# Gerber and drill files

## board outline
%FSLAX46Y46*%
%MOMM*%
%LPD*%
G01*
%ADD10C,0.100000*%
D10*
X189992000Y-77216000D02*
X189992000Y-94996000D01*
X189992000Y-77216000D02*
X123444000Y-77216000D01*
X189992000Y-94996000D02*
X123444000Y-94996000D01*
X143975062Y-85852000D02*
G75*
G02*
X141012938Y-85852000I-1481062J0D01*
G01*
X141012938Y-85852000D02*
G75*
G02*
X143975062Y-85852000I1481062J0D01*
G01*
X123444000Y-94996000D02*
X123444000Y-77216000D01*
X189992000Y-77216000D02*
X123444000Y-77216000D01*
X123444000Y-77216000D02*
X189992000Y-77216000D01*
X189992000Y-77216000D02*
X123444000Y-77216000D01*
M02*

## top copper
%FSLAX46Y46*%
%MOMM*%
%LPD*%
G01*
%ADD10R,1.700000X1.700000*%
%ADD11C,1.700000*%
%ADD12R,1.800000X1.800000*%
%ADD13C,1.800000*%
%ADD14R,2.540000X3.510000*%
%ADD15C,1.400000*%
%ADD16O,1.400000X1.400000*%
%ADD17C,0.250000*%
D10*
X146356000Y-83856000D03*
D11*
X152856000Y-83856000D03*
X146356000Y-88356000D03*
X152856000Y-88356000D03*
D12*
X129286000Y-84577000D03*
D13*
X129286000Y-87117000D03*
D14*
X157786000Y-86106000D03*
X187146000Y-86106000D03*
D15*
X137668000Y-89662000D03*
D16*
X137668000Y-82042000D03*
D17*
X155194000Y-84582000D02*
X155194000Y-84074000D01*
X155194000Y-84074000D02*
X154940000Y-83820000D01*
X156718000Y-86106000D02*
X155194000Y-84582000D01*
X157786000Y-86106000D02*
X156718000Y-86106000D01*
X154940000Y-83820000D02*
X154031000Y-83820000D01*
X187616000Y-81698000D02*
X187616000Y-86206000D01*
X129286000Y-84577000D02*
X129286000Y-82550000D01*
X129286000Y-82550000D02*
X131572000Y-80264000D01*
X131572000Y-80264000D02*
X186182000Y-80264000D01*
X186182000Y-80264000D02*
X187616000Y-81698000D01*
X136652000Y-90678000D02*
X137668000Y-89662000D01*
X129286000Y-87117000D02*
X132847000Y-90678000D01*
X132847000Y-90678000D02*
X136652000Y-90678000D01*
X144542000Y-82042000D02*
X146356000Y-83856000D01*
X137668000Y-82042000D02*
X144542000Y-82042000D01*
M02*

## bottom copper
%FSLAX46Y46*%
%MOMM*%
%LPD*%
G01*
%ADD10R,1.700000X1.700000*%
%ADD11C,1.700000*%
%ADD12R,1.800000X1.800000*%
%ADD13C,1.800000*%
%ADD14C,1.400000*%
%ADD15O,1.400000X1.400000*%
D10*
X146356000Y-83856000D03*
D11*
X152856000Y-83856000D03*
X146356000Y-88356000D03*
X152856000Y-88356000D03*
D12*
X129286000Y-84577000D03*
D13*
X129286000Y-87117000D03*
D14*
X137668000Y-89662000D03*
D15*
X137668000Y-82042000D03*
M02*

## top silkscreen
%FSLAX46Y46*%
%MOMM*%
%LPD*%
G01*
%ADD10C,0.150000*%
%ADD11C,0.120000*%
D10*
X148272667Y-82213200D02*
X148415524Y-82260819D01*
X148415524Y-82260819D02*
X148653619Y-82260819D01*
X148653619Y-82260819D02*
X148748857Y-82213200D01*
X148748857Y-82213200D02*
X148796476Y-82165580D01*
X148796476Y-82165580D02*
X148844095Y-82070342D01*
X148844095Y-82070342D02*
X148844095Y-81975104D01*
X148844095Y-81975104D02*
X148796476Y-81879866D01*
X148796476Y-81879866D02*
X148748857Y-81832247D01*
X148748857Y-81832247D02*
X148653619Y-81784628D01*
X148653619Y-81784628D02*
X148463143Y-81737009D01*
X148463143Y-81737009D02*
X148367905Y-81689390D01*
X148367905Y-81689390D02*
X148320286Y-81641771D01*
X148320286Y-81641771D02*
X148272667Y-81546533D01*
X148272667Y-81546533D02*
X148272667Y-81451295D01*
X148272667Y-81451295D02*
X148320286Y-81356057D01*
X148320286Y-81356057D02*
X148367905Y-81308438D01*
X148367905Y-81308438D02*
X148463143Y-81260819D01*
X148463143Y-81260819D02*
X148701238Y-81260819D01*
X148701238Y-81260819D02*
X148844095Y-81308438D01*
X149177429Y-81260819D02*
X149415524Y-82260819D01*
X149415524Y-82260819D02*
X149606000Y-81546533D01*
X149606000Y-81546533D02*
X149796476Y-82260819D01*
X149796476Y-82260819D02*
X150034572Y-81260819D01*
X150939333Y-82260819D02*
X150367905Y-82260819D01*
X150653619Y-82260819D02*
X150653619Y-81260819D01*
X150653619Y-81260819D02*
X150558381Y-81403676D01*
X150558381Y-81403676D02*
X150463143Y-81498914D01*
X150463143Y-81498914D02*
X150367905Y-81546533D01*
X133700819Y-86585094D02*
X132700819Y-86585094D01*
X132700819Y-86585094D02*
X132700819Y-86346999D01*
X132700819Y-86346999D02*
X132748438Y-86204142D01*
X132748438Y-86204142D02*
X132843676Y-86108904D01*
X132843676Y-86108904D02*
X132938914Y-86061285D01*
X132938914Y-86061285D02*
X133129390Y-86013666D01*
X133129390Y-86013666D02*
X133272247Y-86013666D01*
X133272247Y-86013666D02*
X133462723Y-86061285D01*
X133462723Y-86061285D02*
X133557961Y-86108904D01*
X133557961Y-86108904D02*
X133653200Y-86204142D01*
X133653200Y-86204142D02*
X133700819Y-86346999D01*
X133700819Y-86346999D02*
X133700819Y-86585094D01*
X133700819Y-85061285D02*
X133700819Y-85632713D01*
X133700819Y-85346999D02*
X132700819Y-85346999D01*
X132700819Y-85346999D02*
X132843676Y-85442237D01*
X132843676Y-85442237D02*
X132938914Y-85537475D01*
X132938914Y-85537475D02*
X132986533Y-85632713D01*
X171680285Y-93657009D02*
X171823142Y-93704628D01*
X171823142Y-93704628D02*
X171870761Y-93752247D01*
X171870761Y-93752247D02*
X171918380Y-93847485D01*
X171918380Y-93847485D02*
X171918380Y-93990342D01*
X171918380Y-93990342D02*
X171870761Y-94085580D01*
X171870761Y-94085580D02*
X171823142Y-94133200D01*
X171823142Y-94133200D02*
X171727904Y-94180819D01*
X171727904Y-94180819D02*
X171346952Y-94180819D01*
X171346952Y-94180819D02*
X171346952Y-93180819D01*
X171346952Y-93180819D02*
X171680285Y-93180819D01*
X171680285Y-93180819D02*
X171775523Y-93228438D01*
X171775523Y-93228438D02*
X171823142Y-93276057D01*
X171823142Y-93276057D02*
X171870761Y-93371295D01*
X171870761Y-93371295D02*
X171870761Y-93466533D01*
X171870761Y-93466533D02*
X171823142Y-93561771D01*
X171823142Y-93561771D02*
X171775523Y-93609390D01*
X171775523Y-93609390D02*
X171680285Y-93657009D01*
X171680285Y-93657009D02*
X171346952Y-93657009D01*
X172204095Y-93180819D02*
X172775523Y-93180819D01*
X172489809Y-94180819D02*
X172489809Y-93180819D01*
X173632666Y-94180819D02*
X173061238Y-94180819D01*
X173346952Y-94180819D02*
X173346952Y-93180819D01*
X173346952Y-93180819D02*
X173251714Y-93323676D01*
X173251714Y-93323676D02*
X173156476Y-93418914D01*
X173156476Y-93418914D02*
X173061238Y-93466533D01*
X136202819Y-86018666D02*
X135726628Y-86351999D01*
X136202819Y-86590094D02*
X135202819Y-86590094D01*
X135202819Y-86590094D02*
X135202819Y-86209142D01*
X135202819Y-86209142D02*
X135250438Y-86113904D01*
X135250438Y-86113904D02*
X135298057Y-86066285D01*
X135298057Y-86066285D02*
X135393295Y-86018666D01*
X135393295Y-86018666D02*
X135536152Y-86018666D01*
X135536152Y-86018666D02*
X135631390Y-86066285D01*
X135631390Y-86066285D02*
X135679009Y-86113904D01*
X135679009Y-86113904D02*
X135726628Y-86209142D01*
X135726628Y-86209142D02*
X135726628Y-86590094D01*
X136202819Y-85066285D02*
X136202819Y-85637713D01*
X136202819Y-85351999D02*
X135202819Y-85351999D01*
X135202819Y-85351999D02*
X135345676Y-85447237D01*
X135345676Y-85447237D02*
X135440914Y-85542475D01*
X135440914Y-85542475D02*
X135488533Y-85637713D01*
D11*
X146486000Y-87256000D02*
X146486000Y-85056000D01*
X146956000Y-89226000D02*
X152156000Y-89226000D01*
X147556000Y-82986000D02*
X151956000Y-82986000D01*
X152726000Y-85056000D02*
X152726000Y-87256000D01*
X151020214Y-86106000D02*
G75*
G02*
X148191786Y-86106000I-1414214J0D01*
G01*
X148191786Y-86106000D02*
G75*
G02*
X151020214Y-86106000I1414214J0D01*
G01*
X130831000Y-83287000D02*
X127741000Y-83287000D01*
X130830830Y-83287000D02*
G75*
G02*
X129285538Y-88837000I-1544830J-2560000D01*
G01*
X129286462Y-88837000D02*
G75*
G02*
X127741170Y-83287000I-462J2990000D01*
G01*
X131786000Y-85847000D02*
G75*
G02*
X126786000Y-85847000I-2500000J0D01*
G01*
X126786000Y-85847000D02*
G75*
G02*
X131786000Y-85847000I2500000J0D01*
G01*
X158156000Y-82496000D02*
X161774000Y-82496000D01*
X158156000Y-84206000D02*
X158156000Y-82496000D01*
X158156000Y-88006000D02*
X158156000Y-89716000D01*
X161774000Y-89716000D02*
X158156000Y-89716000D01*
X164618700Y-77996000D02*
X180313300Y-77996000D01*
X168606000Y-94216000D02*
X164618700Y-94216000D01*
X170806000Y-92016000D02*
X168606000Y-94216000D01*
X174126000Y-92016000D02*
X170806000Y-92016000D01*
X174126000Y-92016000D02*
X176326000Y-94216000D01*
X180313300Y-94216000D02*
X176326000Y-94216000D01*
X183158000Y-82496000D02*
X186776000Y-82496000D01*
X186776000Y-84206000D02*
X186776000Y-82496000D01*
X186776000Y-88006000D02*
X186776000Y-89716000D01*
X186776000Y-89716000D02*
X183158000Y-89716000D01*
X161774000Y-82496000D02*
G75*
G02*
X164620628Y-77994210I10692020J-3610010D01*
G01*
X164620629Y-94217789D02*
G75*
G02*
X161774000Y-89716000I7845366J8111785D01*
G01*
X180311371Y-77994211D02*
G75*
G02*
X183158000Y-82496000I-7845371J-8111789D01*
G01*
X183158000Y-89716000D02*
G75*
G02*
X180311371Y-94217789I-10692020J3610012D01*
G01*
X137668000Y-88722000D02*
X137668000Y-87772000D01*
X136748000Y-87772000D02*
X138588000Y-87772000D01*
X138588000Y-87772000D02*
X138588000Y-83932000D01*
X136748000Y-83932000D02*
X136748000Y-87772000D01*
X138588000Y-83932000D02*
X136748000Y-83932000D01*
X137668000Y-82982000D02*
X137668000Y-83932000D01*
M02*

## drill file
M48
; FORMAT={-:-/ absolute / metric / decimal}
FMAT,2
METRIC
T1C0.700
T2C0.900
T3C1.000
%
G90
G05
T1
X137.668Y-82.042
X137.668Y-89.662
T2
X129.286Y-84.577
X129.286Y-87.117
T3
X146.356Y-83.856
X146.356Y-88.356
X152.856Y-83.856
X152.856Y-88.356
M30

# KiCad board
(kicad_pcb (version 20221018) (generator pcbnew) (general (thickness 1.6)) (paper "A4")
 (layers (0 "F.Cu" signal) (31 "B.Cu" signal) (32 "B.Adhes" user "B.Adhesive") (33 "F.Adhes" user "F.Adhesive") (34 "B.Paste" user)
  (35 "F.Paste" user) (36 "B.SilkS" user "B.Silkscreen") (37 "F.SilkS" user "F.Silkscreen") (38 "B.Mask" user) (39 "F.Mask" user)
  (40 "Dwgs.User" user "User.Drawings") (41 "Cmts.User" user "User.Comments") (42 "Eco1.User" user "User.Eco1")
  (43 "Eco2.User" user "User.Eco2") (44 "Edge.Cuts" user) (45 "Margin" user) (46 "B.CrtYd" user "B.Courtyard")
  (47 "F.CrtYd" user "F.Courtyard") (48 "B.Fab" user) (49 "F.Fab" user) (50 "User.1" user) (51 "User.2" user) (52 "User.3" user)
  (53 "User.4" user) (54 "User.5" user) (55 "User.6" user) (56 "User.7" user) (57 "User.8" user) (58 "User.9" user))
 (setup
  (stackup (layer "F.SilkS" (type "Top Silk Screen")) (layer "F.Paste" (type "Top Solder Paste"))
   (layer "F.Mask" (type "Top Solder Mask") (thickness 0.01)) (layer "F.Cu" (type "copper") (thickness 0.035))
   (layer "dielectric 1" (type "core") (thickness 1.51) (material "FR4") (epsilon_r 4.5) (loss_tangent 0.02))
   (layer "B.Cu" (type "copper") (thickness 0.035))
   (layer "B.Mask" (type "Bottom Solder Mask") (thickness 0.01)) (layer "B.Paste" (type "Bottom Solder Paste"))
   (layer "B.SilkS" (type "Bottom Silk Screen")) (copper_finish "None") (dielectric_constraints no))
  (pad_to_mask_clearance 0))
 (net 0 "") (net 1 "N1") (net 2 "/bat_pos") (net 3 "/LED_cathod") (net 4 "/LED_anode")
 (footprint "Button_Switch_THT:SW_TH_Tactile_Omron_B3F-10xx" (layer "F.Cu") (at 146.356 83.856)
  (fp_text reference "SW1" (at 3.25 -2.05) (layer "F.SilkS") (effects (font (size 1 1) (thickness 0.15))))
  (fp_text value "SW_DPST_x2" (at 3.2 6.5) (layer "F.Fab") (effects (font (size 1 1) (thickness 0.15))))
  (fp_line (start 0.13 3.4) (end 0.13 1.2) (stroke (width 0.12) (type solid)) (layer "F.SilkS"))
  (fp_line (start 0.6 5.37) (end 5.8 5.37) (stroke (width 0.12) (type solid)) (layer "F.SilkS"))
  (fp_line (start 1.2 -0.87) (end 5.6 -0.87) (stroke (width 0.12) (type solid)) (layer "F.SilkS"))
  (fp_line (start 6.37 1.2) (end 6.37 3.4) (stroke (width 0.12) (type solid)) (layer "F.SilkS"))
  (fp_circle (center 3.25 2.25) (end 4.25 3.25) (stroke (width 0.12) (type solid)) (fill none) (layer "F.SilkS"))
  (pad "1" thru_hole rect (at 0 0) (size 1.7 1.7) (drill 1) (layers "*.Cu" "*.Mask") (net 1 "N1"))
  (pad "1" thru_hole circle (at 6.5 0) (size 1.7 1.7) (drill 1) (layers "*.Cu" "*.Mask") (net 1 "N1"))
  (pad "2" thru_hole circle (at 0 4.5) (size 1.7 1.7) (drill 1) (layers "*.Cu" "*.Mask") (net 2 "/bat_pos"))
  (pad "2" thru_hole circle (at 6.5 4.5) (size 1.7 1.7) (drill 1) (layers "*.Cu" "*.Mask") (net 2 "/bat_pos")))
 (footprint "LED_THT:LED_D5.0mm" (layer "F.Cu") (at 129.286 84.577 -90)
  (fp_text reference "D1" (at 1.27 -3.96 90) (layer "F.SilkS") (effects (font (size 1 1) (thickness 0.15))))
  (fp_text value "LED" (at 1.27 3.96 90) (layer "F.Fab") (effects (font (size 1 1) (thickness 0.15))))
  (fp_line (start -1.29 -1.545) (end -1.29 1.545) (stroke (width 0.12) (type solid)) (layer "F.SilkS"))
  (fp_arc (start -1.29 -1.54483) (mid 2.072002 -2.880433) (end 4.26 0.000462) (stroke (width 0.12) (type solid)) (layer "F.SilkS"))
  (fp_arc (start 4.26 -0.000462) (mid 2.072002 2.880433) (end -1.29 1.54483) (stroke (width 0.12) (type solid)) (layer "F.SilkS"))
  (fp_circle (center 1.27 0) (end 3.77 0) (stroke (width 0.12) (type solid)) (fill none) (layer "F.SilkS"))
  (pad "1" thru_hole rect (at 0 0 270) (size 1.8 1.8) (drill 0.9) (layers "*.Cu" "*.Mask") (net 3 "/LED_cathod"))
  (pad "2" thru_hole circle (at 2.54 0 270) (size 1.8 1.8) (drill 0.9) (layers "*.Cu" "*.Mask") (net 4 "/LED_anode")))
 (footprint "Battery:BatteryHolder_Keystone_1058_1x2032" (layer "F.Cu") (at 172.466 86.106)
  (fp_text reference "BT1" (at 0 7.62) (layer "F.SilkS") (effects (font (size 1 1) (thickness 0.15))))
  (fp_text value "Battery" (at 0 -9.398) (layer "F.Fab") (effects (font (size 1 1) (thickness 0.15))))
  (fp_line (start -14.31 -3.61) (end -10.692 -3.61) (stroke (width 0.12) (type solid)) (layer "F.SilkS"))
  (fp_line (start -14.31 -1.9) (end -14.31 -3.61) (stroke (width 0.12) (type solid)) (layer "F.SilkS"))
  (fp_line (start -14.31 1.9) (end -14.31 3.61) (stroke (width 0.12) (type solid)) (layer "F.SilkS"))
  (fp_line (start -10.692 3.61) (end -14.31 3.61) (stroke (width 0.12) (type solid)) (layer "F.SilkS"))
  (fp_line (start -7.8473 -8.11) (end 7.8473 -8.11) (stroke (width 0.12) (type solid)) (layer "F.SilkS"))
  (fp_line (start -3.86 8.11) (end -7.8473 8.11) (stroke (width 0.12) (type solid)) (layer "F.SilkS"))
  (fp_line (start -1.66 5.91) (end -3.86 8.11) (stroke (width 0.12) (type solid)) (layer "F.SilkS"))
  (fp_line (start 1.66 5.91) (end -1.66 5.91) (stroke (width 0.12) (type solid)) (layer "F.SilkS"))
  (fp_line (start 1.66 5.91) (end 3.86 8.11) (stroke (width 0.12) (type solid)) (layer "F.SilkS"))
  (fp_line (start 7.8473 8.11) (end 3.86 8.11) (stroke (width 0.12) (type solid)) (layer "F.SilkS"))
  (fp_line (start 10.692 -3.61) (end 14.31 -3.61) (stroke (width 0.12) (type solid)) (layer "F.SilkS"))
  (fp_line (start 14.31 -1.9) (end 14.31 -3.61) (stroke (width 0.12) (type solid)) (layer "F.SilkS"))
  (fp_line (start 14.31 1.9) (end 14.31 3.61) (stroke (width 0.12) (type solid)) (layer "F.SilkS"))
  (fp_line (start 14.31 3.61) (end 10.692 3.61) (stroke (width 0.12) (type solid)) (layer "F.SilkS"))
  (fp_arc (start -10.692 -3.61) (mid -9.538084 -6.031244) (end -7.845371 -8.111789) (stroke (width 0.12) (type solid)) (layer "F.SilkS"))
  (fp_arc (start -7.845371 8.111789) (mid -9.538085 6.031244) (end -10.692 3.61) (stroke (width 0.12) (type solid)) (layer "F.SilkS"))
  (fp_arc (start 7.845371 -8.111789) (mid 9.538085 -6.031244) (end 10.692 -3.61) (stroke (width 0.12) (type solid)) (layer "F.SilkS"))
  (fp_arc (start 10.692 3.61) (mid 9.538084 6.031244) (end 7.845371 8.111789) (stroke (width 0.12) (type solid)) (layer "F.SilkS"))
  (pad "1" smd rect (at -14.68 0) (size 2.54 3.51) (layers "F.Cu" "F.Paste" "F.Mask") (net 2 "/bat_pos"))
  (pad "2" smd rect (at 14.68 0) (size 2.54 3.51) (layers "F.Cu" "F.Paste" "F.Mask") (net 3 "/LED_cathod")))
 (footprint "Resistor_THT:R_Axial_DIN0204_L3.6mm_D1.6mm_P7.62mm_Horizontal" (layer "F.Cu") (at 137.668 89.662 90)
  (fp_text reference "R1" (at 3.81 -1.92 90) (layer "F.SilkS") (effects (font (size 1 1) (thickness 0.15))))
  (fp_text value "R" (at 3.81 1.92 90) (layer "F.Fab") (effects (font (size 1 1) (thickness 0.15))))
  (fp_line (start 0.94 0) (end 1.89 0) (stroke (width 0.12) (type solid)) (layer "F.SilkS"))
  (fp_line (start 1.89 -0.92) (end 1.89 0.92) (stroke (width 0.12) (type solid)) (layer "F.SilkS"))
  (fp_line (start 1.89 0.92) (end 5.73 0.92) (stroke (width 0.12) (type solid)) (layer "F.SilkS"))
  (fp_line (start 5.73 -0.92) (end 1.89 -0.92) (stroke (width 0.12) (type solid)) (layer "F.SilkS"))
  (fp_line (start 5.73 0.92) (end 5.73 -0.92) (stroke (width 0.12) (type solid)) (layer "F.SilkS"))
  (fp_line (start 6.68 0) (end 5.73 0) (stroke (width 0.12) (type solid)) (layer "F.SilkS"))
  (pad "1" thru_hole circle (at 0 0 90) (size 1.4 1.4) (drill 0.7) (layers "*.Cu" "*.Mask") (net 4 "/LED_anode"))
  (pad "2" thru_hole oval (at 7.62 0 90) (size 1.4 1.4) (drill 0.7) (layers "*.Cu" "*.Mask") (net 1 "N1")))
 (gr_line (start 189.992 77.216) (end 189.992 94.996) (stroke (width 0.1) (type default)) (layer "Edge.Cuts"))
 (gr_line (start 189.992 77.216) (end 123.444 77.216) (stroke (width 0.1) (type default)) (layer "Edge.Cuts"))
 (gr_line (start 189.992 94.996) (end 123.444 94.996) (stroke (width 0.1) (type default)) (layer "Edge.Cuts"))
 (gr_circle (center 142.494 85.852) (end 143.764 86.614) (stroke (width 0.1) (type default)) (fill none) (layer "Edge.Cuts"))
 (gr_line (start 123.444 94.996) (end 123.444 77.216) (stroke (width 0.1) (type default)) (layer "Edge.Cuts"))
 (gr_line (start 189.992 77.216) (end 123.444 77.216) (stroke (width 0.1) (type default)) (layer "Edge.Cuts"))
 (gr_line (start 123.444 77.216) (end 189.992 77.216) (stroke (width 0.1) (type default)) (layer "Edge.Cuts"))
 (gr_line (start 189.992 77.216) (end 123.444 77.216) (stroke (width 0.1) (type default)) (layer "Edge.Cuts"))
 (segment (start 155.194 84.582) (end 155.194 84.074) (width 0.25) (layer "F.Cu") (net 2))
 (segment (start 155.194 84.074) (end 154.94 83.82) (width 0.25) (layer "F.Cu") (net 2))
 (segment (start 156.718 86.106) (end 155.194 84.582) (width 0.25) (layer "F.Cu") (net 2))
 (segment (start 157.786 86.106) (end 156.718 86.106) (width 0.25) (layer "F.Cu") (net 2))
 (segment (start 154.94 83.82) (end 154.031 83.82) (width 0.25) (layer "F.Cu") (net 2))
 (segment (start 187.616 81.698) (end 187.616 86.206) (width 0.25) (layer "F.Cu") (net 3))
 (segment (start 129.286 84.577) (end 129.286 82.55) (width 0.25) (layer "F.Cu") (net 3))
 (segment (start 129.286 82.55) (end 131.572 80.264) (width 0.25) (layer "F.Cu") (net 3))
 (segment (start 131.572 80.264) (end 186.182 80.264) (width 0.25) (layer "F.Cu") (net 3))
 (segment (start 186.182 80.264) (end 187.616 81.698) (width 0.25) (layer "F.Cu") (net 3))
 (segment (start 136.652 90.678) (end 137.668 89.662) (width 0.25) (layer "F.Cu") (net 4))
 (segment (start 129.286 87.117) (end 132.847 90.678) (width 0.25) (layer "F.Cu") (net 4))
 (segment (start 132.847 90.678) (end 136.652 90.678) (width 0.25) (layer "F.Cu") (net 4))
 (segment (start 144.542 82.042) (end 146.356 83.856) (width 0.25) (layer "F.Cu") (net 1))
 (segment (start 137.668 82.042) (end 144.542 82.042) (width 0.25) (layer "F.Cu") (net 1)))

